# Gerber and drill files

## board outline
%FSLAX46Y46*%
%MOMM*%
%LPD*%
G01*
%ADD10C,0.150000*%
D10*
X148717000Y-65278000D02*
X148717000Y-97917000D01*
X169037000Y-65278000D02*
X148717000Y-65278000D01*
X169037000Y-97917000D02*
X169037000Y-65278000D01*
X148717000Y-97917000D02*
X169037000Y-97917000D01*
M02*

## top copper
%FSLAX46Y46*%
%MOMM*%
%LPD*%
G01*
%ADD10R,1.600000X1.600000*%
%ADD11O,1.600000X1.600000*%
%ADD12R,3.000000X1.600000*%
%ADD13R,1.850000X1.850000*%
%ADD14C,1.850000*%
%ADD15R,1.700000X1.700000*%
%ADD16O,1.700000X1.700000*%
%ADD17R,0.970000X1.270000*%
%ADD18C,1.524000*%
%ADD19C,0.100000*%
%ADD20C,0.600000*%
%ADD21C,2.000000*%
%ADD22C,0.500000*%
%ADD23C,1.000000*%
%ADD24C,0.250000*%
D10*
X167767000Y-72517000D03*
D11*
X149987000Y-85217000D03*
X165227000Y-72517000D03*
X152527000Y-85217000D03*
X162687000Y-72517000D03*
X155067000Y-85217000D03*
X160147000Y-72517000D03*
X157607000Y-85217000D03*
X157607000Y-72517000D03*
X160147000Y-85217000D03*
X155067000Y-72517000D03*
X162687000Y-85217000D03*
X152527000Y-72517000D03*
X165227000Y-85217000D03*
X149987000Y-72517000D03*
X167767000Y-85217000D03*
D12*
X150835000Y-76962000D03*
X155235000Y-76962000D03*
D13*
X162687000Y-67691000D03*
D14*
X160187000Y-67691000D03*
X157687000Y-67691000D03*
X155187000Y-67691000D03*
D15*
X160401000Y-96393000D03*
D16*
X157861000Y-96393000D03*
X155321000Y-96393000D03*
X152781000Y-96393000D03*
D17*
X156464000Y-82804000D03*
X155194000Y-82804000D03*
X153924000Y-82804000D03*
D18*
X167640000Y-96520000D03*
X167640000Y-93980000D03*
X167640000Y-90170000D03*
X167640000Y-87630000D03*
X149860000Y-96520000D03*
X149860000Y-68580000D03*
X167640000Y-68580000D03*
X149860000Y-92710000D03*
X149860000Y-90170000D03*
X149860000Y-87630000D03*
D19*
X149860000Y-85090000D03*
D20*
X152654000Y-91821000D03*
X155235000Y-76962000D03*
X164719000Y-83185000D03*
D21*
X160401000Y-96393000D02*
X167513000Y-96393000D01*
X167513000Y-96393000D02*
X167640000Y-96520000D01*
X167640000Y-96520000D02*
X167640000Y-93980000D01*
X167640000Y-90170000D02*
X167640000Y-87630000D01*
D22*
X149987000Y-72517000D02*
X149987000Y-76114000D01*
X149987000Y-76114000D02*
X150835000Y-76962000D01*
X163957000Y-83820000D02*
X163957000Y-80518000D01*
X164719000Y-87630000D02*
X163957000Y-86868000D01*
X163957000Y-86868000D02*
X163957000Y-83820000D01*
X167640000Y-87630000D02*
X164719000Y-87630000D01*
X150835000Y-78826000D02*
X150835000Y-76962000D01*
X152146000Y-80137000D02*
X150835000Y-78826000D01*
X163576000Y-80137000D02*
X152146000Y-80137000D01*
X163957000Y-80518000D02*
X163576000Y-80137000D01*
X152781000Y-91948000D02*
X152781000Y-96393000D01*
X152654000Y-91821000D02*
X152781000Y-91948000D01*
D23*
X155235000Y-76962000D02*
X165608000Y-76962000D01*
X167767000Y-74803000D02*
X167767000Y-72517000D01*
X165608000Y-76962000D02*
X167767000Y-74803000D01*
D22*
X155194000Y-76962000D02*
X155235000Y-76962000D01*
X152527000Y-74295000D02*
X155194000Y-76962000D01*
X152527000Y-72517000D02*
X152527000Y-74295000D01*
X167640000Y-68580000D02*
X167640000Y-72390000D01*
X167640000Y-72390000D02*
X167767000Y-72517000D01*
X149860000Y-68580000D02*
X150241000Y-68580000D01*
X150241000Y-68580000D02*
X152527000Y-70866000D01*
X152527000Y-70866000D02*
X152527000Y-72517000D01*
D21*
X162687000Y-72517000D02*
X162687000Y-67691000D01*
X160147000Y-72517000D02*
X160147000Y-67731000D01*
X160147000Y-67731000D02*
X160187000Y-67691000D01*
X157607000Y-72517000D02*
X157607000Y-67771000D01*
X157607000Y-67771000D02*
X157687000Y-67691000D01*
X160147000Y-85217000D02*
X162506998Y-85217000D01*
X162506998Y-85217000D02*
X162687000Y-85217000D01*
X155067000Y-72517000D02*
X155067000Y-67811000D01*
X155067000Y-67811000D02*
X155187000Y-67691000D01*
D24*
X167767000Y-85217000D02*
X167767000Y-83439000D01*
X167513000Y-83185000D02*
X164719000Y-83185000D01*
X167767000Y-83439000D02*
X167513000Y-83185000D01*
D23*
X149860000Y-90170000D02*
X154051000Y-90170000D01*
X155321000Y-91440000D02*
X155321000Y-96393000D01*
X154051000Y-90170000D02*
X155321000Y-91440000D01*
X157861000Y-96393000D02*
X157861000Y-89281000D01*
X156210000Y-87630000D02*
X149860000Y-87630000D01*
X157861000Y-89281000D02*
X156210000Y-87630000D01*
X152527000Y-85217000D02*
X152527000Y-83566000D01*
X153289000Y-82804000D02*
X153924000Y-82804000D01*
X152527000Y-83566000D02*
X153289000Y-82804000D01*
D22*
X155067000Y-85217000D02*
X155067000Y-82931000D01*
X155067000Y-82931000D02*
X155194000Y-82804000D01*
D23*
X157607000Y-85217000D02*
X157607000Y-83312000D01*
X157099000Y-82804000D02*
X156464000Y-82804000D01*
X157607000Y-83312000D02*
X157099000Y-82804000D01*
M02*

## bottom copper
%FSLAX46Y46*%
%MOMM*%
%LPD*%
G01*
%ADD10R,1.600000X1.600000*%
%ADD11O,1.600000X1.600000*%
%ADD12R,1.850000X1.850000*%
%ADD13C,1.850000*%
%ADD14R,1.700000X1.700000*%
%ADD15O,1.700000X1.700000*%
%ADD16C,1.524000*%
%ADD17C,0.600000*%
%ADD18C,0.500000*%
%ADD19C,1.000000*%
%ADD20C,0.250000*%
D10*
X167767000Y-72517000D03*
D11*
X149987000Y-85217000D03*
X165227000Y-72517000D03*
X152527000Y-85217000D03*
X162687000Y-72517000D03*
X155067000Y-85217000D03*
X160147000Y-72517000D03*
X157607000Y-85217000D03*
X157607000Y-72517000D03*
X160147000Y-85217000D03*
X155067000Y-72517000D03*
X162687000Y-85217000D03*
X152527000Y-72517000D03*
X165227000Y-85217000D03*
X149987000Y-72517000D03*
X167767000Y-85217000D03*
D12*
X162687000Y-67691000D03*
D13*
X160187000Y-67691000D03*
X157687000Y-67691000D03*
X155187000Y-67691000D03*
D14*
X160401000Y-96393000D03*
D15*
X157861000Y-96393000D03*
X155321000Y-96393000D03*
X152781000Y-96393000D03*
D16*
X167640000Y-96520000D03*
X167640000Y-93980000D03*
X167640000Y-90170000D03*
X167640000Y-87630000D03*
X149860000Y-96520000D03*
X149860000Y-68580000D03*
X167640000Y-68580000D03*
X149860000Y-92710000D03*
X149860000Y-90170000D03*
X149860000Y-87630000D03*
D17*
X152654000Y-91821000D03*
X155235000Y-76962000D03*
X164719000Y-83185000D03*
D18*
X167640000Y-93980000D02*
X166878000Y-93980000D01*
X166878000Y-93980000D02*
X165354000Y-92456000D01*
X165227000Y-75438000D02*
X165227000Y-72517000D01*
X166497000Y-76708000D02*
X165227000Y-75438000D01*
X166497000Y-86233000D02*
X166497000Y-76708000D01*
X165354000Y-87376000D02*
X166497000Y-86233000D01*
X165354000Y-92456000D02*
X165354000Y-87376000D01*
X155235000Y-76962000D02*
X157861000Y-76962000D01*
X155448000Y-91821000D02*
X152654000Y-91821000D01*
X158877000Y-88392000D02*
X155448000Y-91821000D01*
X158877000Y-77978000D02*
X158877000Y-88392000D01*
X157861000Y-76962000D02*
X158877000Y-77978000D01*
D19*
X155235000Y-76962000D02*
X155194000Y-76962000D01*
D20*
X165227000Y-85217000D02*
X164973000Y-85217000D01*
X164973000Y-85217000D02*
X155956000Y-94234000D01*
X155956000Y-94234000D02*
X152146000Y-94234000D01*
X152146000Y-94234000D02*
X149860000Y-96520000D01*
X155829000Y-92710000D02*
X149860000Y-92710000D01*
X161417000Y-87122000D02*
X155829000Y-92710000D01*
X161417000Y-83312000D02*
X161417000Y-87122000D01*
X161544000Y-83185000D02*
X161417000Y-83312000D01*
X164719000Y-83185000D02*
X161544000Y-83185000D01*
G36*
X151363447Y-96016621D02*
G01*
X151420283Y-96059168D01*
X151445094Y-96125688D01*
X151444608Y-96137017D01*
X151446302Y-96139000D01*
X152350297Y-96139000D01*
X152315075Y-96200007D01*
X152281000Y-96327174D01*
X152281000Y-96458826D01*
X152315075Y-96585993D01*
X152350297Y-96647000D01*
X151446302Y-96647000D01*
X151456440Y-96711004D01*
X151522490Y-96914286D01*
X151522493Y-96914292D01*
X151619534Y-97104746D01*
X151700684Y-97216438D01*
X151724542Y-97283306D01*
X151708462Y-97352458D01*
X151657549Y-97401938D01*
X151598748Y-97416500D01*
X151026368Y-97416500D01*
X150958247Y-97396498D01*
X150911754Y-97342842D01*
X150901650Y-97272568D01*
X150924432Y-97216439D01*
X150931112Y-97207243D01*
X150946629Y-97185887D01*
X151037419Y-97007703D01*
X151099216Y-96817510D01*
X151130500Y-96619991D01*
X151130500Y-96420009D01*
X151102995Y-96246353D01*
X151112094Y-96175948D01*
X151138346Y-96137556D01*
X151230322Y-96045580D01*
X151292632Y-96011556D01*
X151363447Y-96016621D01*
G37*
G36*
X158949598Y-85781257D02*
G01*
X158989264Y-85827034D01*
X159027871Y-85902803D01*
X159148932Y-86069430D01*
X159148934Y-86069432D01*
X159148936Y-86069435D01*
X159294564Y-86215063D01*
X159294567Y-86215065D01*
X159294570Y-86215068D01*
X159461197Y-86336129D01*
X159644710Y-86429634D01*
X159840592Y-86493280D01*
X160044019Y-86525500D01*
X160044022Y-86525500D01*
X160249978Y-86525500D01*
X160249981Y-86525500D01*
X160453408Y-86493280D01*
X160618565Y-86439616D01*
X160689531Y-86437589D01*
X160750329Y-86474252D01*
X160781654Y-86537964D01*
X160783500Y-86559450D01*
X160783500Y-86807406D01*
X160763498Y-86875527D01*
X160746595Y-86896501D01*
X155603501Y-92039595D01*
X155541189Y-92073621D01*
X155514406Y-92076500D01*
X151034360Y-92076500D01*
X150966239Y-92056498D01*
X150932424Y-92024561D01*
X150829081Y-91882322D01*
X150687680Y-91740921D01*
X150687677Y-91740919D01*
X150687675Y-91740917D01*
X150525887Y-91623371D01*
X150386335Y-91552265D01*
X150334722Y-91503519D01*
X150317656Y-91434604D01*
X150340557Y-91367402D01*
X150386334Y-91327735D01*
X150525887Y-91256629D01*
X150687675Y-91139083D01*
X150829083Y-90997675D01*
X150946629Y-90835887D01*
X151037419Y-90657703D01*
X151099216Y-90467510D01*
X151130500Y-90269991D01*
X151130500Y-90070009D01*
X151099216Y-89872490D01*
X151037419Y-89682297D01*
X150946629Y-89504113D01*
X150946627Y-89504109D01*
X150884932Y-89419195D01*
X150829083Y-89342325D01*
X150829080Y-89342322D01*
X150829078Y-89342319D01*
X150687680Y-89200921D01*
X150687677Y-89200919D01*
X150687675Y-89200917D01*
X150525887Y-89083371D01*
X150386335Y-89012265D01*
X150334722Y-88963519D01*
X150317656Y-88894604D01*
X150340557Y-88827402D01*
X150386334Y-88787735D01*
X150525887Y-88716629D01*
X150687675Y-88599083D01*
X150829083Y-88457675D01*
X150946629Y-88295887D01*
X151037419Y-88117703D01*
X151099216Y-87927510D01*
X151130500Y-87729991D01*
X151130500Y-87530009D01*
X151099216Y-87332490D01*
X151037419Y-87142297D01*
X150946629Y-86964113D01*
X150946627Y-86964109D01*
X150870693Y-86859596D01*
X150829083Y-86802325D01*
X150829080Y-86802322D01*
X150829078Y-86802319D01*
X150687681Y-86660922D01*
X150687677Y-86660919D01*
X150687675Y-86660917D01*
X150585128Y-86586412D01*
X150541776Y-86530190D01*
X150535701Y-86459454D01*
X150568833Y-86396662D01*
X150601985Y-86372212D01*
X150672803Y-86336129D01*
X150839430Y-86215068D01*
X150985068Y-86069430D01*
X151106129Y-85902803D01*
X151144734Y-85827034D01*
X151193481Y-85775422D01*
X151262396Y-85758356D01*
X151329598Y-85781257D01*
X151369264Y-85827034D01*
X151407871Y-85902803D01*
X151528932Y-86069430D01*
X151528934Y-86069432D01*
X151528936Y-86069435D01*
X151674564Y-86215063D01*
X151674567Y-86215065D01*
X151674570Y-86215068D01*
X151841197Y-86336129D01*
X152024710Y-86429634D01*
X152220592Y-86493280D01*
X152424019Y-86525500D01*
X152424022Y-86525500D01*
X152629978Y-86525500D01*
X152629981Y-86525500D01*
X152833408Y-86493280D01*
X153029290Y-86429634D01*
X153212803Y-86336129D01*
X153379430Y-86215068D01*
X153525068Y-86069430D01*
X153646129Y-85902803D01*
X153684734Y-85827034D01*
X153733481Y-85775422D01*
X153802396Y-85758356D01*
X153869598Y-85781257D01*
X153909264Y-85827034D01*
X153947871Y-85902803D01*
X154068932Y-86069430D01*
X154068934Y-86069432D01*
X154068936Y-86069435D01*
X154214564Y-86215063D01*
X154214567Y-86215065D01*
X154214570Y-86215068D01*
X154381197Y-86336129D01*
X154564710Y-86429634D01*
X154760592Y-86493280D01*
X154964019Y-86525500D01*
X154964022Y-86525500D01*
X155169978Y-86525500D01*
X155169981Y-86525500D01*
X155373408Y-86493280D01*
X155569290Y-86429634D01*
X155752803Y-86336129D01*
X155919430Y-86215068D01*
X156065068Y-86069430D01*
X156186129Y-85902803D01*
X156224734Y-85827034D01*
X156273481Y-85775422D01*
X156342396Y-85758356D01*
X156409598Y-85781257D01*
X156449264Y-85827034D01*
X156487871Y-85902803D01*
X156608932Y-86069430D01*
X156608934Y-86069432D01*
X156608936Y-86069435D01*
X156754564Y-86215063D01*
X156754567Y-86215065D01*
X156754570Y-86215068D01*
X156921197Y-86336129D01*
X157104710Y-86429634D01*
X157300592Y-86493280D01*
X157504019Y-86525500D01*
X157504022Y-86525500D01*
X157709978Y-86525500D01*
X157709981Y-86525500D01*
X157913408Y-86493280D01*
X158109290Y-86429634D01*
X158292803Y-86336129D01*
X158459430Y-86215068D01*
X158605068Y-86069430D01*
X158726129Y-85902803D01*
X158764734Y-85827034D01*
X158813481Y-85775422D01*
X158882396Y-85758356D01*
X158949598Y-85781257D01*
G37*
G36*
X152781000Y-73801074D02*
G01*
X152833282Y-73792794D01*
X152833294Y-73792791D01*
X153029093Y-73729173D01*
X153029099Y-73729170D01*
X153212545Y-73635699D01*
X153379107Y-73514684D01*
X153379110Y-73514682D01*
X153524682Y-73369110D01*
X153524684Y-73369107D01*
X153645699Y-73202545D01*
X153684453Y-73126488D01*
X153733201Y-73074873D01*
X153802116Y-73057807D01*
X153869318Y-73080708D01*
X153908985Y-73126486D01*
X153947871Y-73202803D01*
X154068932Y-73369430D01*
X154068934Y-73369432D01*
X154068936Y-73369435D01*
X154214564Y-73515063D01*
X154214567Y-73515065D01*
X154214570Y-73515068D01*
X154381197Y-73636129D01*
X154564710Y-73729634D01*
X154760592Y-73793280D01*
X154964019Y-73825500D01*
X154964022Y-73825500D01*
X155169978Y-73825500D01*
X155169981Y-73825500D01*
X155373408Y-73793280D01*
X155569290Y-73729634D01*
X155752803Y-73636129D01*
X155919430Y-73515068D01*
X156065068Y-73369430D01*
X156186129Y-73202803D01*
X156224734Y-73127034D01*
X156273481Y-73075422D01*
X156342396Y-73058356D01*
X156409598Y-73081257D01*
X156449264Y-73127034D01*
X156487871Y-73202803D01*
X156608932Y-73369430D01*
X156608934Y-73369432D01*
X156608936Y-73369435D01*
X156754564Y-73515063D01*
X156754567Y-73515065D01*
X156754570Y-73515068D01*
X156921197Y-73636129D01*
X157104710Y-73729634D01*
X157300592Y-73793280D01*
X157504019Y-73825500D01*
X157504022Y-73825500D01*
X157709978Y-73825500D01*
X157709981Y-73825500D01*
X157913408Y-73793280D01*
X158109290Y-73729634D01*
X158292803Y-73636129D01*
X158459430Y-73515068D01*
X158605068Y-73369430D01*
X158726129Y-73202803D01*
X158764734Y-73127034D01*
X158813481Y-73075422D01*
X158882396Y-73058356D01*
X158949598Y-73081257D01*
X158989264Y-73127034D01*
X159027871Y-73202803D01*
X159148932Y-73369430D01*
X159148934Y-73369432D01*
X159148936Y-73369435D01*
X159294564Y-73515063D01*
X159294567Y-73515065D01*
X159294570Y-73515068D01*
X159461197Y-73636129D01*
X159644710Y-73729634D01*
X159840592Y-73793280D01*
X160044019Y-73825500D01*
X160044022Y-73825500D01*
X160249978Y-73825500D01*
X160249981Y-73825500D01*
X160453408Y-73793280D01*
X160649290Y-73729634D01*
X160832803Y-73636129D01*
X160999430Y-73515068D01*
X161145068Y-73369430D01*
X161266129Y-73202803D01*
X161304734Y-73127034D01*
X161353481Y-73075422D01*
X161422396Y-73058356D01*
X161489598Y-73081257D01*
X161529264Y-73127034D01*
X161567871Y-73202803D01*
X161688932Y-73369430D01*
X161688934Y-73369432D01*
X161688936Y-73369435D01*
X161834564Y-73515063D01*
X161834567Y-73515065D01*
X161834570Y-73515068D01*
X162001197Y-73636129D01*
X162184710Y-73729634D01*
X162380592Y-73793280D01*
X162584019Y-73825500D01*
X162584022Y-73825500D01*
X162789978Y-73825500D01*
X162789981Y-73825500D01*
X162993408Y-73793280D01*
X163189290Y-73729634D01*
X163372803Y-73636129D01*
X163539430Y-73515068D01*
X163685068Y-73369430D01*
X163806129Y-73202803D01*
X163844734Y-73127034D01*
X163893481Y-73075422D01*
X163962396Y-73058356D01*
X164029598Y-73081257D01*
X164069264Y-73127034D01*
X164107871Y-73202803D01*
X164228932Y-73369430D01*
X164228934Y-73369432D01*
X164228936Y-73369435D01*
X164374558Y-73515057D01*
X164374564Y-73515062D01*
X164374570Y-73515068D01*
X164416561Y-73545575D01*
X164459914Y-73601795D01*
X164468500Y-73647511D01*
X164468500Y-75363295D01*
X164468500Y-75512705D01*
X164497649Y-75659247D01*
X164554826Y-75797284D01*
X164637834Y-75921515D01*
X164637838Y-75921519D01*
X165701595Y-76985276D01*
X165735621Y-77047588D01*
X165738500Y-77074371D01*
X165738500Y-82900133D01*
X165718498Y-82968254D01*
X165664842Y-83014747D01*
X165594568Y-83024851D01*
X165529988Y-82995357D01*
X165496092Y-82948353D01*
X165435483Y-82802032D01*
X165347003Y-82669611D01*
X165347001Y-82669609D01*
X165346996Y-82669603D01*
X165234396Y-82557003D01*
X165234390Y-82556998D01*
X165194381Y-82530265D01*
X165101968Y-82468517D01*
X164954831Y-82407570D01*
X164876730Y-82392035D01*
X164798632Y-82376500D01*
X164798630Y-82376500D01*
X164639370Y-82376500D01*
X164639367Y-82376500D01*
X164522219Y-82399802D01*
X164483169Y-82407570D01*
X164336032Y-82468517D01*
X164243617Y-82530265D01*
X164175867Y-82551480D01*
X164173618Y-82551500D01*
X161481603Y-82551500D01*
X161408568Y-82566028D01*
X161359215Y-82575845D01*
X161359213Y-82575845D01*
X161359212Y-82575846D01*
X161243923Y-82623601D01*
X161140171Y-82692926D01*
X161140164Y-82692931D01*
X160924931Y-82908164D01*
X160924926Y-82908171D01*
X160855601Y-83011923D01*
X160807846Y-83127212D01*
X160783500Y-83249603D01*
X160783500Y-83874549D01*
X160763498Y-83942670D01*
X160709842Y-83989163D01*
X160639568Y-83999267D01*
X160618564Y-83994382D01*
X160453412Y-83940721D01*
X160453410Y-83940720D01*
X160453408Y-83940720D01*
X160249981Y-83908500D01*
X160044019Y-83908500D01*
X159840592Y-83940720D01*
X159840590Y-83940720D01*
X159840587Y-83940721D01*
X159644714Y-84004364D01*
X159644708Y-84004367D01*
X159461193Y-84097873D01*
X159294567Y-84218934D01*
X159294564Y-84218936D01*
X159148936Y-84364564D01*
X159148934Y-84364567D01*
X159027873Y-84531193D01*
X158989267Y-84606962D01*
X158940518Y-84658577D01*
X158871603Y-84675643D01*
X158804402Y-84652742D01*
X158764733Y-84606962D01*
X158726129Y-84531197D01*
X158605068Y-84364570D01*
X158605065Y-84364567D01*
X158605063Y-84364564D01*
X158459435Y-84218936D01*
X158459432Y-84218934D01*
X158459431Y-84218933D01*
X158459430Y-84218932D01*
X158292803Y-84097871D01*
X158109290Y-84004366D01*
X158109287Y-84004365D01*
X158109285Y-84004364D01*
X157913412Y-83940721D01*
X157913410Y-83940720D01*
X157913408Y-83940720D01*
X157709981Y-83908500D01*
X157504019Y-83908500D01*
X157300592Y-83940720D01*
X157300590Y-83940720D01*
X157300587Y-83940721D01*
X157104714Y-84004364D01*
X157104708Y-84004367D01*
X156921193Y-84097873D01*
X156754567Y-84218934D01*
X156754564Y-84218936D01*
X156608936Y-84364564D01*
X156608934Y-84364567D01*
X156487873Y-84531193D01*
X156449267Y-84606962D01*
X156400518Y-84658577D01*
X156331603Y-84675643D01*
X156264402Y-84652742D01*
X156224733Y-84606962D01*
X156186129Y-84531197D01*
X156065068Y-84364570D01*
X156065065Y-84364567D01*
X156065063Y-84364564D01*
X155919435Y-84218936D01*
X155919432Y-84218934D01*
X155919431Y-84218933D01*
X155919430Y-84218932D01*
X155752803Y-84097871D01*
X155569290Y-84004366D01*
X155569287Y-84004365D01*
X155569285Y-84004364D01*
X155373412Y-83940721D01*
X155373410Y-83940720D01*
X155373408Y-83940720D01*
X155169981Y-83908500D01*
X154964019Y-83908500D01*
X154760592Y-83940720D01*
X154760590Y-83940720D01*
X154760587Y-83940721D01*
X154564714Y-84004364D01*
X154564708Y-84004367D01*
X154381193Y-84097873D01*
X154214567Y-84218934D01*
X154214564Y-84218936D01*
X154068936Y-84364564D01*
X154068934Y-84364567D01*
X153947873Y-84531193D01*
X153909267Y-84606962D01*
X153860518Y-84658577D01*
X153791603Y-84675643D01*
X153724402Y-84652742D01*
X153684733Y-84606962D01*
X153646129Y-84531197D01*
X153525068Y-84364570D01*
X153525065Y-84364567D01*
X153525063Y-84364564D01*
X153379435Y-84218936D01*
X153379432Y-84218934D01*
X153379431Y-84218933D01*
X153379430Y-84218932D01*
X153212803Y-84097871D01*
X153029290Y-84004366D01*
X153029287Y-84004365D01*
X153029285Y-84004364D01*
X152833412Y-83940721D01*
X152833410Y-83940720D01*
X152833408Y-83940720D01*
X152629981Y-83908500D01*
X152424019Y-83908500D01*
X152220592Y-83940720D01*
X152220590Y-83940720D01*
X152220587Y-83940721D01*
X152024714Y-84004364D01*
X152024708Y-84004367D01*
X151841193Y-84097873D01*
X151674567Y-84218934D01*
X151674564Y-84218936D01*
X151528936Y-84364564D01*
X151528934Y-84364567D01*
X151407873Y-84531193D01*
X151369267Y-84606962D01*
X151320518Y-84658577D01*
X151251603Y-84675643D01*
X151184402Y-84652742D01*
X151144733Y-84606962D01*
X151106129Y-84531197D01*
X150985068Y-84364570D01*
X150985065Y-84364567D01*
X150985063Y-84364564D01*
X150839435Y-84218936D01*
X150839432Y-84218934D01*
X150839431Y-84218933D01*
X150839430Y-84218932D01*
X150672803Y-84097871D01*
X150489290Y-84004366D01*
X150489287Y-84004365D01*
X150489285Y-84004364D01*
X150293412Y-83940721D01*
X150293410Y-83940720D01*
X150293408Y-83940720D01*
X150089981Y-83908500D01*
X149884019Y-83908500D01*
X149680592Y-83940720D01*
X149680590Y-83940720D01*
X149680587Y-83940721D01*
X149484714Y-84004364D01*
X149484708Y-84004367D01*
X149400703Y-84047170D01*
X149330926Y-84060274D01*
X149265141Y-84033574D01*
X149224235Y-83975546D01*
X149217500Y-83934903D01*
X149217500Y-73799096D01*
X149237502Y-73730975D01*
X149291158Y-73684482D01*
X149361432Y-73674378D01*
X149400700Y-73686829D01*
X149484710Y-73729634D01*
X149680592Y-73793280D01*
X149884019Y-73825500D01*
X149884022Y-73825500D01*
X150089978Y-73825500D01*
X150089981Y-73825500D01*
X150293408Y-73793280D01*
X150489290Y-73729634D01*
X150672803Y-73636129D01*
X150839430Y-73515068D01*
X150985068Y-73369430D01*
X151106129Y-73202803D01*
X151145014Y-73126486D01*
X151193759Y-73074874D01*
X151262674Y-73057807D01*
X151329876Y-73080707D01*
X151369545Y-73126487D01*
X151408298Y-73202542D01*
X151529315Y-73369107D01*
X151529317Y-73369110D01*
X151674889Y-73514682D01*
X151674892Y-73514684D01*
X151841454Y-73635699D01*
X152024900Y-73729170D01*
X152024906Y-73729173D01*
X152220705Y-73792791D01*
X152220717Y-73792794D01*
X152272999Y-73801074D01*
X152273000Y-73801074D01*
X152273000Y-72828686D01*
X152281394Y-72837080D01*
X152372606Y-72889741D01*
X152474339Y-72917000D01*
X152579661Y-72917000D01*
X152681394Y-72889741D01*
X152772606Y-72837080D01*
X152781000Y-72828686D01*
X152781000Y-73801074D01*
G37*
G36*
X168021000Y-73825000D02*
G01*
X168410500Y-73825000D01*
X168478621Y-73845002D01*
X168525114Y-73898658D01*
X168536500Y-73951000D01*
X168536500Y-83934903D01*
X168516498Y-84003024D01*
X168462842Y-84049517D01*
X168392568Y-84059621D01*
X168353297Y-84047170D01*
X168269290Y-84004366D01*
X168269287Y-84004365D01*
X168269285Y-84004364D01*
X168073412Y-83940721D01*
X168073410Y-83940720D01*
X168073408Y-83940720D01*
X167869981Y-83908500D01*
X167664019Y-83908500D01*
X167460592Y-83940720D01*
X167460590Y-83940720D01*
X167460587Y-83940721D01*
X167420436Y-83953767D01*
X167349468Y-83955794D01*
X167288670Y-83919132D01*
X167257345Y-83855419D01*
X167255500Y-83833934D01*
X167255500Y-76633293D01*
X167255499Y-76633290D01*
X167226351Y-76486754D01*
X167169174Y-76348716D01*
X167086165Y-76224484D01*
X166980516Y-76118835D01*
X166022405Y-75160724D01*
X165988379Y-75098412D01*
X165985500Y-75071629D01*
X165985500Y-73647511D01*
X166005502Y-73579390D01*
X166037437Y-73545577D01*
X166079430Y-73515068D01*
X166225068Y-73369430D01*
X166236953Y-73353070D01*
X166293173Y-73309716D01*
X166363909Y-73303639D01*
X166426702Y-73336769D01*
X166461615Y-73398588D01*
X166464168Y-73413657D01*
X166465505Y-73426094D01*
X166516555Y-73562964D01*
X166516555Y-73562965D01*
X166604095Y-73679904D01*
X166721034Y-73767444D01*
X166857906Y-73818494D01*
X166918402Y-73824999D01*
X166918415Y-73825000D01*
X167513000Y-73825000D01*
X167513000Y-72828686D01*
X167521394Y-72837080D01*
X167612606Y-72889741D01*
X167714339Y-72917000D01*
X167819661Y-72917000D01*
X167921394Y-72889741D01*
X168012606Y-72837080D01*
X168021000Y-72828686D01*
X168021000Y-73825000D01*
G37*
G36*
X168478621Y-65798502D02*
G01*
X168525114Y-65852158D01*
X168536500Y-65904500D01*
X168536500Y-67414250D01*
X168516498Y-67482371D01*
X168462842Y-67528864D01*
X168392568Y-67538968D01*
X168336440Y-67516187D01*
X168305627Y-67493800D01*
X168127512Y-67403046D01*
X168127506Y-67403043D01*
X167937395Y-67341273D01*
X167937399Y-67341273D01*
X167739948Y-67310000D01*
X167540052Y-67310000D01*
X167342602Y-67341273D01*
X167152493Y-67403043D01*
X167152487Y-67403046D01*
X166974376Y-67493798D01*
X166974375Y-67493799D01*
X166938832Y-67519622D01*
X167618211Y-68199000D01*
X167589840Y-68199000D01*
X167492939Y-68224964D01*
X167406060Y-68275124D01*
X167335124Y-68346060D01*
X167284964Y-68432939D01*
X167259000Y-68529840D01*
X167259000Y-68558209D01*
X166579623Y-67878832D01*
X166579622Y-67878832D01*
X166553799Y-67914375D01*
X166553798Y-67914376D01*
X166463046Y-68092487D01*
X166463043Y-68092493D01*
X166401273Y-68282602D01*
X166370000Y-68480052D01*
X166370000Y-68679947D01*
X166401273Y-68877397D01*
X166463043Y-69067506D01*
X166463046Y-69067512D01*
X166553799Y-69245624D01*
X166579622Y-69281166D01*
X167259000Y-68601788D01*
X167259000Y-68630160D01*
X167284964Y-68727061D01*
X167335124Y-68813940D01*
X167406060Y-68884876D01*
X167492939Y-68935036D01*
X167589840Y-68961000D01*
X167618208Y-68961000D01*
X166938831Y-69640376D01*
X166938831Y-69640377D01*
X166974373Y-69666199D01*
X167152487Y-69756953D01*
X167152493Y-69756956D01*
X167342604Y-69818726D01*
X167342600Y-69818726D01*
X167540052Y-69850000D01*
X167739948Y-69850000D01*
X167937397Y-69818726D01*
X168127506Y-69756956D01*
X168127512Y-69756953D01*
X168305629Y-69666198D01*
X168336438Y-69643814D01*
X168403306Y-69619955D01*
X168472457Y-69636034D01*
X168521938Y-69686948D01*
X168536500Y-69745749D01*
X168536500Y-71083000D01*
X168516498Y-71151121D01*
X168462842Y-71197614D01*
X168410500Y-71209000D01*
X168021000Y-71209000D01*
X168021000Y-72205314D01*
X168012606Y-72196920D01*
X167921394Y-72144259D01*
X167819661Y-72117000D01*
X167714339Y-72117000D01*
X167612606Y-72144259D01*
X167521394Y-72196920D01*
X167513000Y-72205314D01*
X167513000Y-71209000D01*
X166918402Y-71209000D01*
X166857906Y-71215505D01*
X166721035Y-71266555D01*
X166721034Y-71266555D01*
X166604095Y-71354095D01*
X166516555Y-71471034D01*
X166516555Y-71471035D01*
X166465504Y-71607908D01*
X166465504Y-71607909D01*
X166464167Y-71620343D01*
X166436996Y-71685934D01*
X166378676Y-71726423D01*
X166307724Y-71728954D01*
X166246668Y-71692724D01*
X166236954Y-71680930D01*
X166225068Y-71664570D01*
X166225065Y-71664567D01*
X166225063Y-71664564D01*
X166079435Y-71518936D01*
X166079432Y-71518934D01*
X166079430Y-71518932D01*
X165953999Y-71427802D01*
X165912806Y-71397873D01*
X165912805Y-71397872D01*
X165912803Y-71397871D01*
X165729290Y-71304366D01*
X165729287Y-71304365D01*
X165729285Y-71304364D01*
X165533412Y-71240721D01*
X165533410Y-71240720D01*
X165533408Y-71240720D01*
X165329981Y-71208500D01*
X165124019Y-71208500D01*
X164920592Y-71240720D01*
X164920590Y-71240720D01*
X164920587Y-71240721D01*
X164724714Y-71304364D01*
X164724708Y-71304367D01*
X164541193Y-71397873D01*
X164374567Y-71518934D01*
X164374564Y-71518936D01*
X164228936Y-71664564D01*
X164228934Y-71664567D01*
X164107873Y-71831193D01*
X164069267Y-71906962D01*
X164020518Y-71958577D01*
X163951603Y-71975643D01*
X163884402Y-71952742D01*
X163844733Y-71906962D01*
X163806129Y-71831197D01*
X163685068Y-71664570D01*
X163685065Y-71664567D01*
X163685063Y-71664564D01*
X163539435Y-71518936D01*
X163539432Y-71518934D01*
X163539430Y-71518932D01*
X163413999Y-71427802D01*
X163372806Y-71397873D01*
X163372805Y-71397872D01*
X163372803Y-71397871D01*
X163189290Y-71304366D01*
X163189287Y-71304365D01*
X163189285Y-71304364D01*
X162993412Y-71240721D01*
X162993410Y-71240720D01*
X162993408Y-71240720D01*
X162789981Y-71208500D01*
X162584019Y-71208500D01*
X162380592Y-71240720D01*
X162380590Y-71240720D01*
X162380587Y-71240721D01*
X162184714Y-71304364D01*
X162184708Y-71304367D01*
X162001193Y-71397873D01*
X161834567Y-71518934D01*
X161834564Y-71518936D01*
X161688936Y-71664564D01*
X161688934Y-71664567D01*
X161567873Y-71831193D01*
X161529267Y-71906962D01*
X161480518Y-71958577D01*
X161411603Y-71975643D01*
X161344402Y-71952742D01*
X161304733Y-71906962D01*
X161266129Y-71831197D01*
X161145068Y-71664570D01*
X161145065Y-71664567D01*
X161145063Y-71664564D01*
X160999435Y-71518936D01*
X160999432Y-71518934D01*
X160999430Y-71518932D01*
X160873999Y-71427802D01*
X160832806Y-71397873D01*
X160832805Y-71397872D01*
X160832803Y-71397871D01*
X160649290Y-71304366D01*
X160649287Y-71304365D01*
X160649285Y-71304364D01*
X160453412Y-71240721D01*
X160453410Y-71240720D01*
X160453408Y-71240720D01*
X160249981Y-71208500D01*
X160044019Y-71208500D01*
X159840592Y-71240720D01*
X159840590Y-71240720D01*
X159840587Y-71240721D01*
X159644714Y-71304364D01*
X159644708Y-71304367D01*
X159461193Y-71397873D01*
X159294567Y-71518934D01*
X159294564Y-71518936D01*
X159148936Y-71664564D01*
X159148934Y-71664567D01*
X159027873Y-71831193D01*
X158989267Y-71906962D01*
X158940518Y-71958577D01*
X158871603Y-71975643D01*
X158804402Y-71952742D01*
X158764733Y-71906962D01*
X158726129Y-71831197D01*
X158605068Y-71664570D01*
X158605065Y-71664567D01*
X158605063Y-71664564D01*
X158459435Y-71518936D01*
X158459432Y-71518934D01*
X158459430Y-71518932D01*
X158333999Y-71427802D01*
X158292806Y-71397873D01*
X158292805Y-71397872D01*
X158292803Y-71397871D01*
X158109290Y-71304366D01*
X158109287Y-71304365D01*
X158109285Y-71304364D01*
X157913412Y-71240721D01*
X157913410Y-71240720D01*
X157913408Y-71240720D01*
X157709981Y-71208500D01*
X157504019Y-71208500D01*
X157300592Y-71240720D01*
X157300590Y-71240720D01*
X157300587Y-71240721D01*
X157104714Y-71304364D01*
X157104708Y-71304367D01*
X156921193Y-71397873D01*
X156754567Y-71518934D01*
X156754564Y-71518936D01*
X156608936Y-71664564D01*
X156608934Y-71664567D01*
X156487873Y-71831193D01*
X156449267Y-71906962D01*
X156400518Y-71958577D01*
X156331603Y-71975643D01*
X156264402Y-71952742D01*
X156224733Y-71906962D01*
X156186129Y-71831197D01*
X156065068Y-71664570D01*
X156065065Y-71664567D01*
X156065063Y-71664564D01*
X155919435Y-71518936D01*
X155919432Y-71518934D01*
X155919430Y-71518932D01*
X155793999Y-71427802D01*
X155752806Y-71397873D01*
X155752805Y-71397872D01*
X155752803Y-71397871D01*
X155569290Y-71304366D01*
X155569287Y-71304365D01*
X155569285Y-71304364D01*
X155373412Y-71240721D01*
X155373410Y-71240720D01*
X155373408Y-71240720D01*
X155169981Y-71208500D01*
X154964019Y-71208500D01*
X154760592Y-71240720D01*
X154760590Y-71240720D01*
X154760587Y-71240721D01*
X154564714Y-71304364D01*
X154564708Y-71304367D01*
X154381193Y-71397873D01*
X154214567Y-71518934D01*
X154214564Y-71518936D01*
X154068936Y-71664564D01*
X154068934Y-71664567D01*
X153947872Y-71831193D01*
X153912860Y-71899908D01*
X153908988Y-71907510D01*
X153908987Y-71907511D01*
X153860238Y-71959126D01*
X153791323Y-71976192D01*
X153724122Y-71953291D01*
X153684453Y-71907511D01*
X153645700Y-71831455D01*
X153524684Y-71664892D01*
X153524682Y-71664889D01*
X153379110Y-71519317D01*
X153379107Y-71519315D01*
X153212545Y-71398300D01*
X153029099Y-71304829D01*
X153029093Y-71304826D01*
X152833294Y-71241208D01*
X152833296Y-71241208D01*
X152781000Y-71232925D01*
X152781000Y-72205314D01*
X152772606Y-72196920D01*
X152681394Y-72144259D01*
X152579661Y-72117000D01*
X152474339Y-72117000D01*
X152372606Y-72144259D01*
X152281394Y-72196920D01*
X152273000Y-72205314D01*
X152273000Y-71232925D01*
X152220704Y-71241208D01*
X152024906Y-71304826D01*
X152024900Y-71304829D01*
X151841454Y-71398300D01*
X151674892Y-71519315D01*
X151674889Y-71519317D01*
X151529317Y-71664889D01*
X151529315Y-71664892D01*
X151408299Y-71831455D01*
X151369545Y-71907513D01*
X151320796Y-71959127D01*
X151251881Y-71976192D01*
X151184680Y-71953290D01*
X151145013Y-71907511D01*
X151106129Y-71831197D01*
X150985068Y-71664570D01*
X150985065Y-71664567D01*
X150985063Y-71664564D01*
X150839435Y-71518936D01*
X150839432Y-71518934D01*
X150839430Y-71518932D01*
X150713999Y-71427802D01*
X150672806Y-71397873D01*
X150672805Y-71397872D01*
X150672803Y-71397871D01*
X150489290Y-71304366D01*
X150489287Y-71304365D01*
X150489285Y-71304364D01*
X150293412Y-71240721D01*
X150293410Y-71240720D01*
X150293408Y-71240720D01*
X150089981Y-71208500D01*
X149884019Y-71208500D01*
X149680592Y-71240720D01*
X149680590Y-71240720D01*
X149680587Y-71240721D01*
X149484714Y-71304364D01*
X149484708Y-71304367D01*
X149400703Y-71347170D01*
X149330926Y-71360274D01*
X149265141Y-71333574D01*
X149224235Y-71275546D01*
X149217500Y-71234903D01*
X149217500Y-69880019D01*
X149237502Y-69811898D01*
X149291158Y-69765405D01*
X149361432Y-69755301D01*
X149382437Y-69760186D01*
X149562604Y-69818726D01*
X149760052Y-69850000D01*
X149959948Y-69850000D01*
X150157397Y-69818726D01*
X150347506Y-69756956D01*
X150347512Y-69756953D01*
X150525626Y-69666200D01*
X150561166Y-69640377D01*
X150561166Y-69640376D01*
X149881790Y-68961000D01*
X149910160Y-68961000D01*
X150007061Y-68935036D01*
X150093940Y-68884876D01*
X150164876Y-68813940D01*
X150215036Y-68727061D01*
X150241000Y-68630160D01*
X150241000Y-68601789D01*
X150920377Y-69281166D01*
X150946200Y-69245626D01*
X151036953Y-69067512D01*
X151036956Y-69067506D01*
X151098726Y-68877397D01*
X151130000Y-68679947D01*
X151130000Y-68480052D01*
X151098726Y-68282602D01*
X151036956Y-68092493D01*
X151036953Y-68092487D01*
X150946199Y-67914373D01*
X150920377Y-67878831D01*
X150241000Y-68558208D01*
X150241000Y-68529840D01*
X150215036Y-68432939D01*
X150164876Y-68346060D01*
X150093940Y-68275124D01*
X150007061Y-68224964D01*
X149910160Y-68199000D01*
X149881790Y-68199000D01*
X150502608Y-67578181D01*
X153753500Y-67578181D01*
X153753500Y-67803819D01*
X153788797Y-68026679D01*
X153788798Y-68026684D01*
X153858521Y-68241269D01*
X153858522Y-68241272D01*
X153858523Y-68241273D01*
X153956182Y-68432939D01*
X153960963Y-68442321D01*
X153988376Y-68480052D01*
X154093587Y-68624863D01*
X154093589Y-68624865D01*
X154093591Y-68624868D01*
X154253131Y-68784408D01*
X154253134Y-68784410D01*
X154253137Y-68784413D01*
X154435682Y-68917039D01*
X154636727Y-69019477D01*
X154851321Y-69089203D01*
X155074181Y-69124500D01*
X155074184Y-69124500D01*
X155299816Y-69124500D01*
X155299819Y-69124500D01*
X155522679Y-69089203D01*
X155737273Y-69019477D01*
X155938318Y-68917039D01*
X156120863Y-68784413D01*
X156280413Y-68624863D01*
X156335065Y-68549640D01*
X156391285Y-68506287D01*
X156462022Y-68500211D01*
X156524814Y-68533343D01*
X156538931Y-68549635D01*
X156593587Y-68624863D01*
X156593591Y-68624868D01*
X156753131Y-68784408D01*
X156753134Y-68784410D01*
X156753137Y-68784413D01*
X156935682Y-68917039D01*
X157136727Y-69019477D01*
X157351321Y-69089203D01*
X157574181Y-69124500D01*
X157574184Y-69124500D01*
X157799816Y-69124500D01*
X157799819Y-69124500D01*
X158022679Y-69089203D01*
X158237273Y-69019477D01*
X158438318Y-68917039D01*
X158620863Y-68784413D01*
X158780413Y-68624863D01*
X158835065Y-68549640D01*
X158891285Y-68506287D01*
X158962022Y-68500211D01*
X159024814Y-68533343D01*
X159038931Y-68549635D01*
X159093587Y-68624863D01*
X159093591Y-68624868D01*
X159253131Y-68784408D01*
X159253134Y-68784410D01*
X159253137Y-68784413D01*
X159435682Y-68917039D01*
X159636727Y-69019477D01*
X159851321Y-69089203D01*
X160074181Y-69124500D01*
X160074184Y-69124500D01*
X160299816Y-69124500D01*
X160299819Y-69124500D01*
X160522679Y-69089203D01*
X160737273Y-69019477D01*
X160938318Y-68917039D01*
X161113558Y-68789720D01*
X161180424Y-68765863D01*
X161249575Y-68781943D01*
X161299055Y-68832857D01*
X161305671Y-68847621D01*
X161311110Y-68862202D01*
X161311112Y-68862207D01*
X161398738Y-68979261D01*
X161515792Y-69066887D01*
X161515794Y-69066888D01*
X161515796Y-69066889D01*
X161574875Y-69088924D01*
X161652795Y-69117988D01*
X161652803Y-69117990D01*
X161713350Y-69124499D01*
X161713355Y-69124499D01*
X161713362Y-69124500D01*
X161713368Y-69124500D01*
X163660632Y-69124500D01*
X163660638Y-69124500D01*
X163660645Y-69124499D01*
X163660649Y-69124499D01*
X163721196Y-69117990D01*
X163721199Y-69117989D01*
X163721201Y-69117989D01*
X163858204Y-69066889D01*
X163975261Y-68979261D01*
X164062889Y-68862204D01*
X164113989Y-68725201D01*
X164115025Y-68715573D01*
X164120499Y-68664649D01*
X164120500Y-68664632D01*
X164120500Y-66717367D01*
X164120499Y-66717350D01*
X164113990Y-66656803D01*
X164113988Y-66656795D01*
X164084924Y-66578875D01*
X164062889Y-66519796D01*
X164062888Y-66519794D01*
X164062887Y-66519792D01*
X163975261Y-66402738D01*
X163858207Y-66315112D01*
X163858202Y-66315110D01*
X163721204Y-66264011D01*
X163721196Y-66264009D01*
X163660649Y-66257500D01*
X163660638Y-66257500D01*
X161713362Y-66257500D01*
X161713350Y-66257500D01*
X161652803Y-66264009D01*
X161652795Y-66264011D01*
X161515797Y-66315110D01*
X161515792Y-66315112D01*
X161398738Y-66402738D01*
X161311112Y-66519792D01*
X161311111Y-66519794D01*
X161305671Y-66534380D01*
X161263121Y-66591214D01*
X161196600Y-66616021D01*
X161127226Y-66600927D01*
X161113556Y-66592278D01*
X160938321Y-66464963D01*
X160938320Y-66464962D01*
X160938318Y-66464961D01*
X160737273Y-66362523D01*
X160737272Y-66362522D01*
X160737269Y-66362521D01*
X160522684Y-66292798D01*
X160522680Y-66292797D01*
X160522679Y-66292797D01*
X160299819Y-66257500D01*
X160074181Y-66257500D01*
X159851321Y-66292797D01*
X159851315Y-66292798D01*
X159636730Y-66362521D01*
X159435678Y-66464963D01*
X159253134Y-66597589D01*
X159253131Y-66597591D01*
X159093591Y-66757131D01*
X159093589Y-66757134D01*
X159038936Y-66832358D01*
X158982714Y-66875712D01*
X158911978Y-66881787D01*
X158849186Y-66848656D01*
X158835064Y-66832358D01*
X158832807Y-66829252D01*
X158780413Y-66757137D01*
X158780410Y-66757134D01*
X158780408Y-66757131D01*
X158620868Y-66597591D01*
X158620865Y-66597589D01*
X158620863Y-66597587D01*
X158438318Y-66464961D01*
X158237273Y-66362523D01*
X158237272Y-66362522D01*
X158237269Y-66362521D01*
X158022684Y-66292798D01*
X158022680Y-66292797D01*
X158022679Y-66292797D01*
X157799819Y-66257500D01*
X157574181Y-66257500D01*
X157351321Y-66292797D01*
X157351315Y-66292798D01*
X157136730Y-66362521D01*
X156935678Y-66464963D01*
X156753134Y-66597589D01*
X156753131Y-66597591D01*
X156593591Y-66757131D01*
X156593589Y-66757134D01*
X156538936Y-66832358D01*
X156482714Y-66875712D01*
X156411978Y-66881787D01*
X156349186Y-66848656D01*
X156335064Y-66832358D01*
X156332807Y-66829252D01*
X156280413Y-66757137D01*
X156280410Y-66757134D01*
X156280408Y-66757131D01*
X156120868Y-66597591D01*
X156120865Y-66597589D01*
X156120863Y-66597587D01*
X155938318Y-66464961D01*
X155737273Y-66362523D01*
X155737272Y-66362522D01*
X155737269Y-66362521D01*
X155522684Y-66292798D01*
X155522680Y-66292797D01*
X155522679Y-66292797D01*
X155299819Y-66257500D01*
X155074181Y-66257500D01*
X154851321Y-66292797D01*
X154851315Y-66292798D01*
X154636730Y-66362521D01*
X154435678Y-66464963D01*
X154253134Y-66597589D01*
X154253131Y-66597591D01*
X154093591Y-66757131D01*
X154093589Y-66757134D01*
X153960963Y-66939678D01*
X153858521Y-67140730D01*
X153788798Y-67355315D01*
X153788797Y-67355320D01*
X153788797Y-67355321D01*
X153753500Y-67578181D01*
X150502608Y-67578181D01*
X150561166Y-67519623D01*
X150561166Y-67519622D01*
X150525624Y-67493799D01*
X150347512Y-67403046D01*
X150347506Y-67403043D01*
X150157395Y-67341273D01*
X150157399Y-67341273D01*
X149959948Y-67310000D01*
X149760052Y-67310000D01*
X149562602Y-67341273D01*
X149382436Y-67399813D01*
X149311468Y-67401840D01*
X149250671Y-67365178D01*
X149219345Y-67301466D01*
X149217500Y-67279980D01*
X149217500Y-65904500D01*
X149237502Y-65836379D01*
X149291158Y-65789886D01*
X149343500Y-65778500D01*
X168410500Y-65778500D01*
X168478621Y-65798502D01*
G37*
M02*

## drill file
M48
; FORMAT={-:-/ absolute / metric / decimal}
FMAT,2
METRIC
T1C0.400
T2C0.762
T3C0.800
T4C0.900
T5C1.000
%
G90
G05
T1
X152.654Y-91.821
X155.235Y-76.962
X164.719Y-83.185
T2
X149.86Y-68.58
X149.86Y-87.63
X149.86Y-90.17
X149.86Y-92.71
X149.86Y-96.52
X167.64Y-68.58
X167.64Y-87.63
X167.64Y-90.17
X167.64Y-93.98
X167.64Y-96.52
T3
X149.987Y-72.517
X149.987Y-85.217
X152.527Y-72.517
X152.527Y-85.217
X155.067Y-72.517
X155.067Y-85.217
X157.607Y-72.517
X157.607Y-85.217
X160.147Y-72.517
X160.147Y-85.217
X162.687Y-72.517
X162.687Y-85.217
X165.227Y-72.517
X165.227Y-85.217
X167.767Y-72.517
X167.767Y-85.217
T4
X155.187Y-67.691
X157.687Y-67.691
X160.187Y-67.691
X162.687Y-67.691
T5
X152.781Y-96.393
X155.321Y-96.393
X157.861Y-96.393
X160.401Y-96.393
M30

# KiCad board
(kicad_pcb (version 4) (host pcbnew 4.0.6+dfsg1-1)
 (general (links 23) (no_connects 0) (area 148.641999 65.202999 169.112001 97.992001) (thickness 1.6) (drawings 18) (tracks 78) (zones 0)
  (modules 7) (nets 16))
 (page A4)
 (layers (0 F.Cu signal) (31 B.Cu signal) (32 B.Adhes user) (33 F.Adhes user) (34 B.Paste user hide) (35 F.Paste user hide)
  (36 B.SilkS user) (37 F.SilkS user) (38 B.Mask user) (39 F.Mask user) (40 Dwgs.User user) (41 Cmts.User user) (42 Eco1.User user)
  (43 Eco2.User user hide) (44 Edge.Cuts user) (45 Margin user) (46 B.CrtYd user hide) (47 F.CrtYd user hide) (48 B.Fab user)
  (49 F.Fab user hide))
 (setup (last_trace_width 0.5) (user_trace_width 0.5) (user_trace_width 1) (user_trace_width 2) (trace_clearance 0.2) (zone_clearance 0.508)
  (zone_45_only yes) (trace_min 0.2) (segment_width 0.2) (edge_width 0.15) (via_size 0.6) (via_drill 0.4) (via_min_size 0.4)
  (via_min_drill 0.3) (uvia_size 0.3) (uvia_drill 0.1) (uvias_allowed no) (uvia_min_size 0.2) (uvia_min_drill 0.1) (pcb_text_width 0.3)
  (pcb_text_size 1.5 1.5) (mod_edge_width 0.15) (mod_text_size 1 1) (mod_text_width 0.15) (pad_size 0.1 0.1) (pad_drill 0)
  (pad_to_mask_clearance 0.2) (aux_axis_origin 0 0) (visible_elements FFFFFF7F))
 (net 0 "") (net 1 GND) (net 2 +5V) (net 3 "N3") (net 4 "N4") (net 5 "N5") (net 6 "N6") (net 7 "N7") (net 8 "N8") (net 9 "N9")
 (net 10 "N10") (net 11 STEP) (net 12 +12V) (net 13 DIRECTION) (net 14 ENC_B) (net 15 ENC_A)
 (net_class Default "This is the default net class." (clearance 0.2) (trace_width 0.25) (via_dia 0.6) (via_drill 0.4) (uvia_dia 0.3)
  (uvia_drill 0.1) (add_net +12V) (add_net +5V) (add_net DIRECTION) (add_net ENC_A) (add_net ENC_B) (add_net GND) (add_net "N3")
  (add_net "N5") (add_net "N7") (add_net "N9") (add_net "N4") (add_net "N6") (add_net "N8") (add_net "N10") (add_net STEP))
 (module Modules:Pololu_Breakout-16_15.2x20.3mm (layer F.Cu) (at 167.767 72.517 270)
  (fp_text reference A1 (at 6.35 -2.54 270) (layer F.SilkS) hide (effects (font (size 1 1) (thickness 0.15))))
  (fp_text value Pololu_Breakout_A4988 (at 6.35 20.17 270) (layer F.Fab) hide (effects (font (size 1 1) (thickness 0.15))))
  (pad 1 thru_hole rect (at 0 0 270) (size 1.6 1.6) (drill 0.8) (layers *.Cu *.Mask) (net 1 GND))
  (pad 9 thru_hole oval (at 12.7 17.78 270) (size 1.6 1.6) (drill 0.8) (layers *.Cu *.Mask))
  (pad 2 thru_hole oval (at 0 2.54 270) (size 1.6 1.6) (drill 0.8) (layers *.Cu *.Mask) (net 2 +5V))
  (pad 10 thru_hole oval (at 12.7 15.24 270) (size 1.6 1.6) (drill 0.8) (layers *.Cu *.Mask) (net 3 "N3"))
  (pad 3 thru_hole oval (at 0 5.08 270) (size 1.6 1.6) (drill 0.8) (layers *.Cu *.Mask) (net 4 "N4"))
  (pad 11 thru_hole oval (at 12.7 12.7 270) (size 1.6 1.6) (drill 0.8) (layers *.Cu *.Mask) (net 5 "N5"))
  (pad 4 thru_hole oval (at 0 7.62 270) (size 1.6 1.6) (drill 0.8) (layers *.Cu *.Mask) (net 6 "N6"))
  (pad 12 thru_hole oval (at 12.7 10.16 270) (size 1.6 1.6) (drill 0.8) (layers *.Cu *.Mask) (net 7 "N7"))
  (pad 5 thru_hole oval (at 0 10.16 270) (size 1.6 1.6) (drill 0.8) (layers *.Cu *.Mask) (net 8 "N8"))
  (pad 13 thru_hole oval (at 12.7 7.62 270) (size 1.6 1.6) (drill 0.8) (layers *.Cu *.Mask) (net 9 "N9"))
  (pad 6 thru_hole oval (at 0 12.7 270) (size 1.6 1.6) (drill 0.8) (layers *.Cu *.Mask) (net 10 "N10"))
  (pad 14 thru_hole oval (at 12.7 5.08 270) (size 1.6 1.6) (drill 0.8) (layers *.Cu *.Mask) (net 9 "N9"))
  (pad 7 thru_hole oval (at 0 15.24 270) (size 1.6 1.6) (drill 0.8) (layers *.Cu *.Mask) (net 1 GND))
  (pad 15 thru_hole oval (at 12.7 2.54 270) (size 1.6 1.6) (drill 0.8) (layers *.Cu *.Mask) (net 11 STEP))
  (pad 8 thru_hole oval (at 0 17.78 270) (size 1.6 1.6) (drill 0.8) (layers *.Cu *.Mask) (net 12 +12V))
  (pad 16 thru_hole oval (at 12.7 0 270) (size 1.6 1.6) (drill 0.8) (layers *.Cu *.Mask) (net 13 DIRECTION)))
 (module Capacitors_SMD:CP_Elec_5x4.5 (layer F.Cu) (at 153.035 76.962)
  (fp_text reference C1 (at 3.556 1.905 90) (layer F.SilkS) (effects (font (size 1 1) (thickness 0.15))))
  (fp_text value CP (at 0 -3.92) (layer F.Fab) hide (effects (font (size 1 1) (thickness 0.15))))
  (pad 1 smd rect (at -2.2 0 180) (size 3 1.6) (layers F.Cu F.Paste F.Mask) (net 12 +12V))
  (pad 2 smd rect (at 2.2 0 180) (size 3 1.6) (layers F.Cu F.Paste F.Mask) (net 1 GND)))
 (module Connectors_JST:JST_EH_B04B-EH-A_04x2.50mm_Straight (layer F.Cu) (at 162.687 67.691 180)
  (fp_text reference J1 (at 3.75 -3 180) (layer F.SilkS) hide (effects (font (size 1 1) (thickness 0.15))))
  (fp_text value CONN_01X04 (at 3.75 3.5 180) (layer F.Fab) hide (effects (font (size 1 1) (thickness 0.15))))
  (pad 1 thru_hole rect (at 0 0 180) (size 1.85 1.85) (drill 0.9) (layers *.Cu *.Mask) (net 4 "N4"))
  (pad 2 thru_hole circle (at 2.5 0 180) (size 1.85 1.85) (drill 0.9) (layers *.Cu *.Mask) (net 6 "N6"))
  (pad 3 thru_hole circle (at 5 0 180) (size 1.85 1.85) (drill 0.9) (layers *.Cu *.Mask) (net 8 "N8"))
  (pad 4 thru_hole circle (at 7.5 0 180) (size 1.85 1.85) (drill 0.9) (layers *.Cu *.Mask) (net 10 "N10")))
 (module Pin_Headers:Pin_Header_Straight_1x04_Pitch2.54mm (layer F.Cu) (at 160.401 96.393 270)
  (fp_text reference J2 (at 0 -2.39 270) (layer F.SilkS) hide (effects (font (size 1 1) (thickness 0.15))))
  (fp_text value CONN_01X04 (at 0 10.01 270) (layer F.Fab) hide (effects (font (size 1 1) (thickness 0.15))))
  (pad 1 thru_hole rect (at 0 0 270) (size 1.7 1.7) (drill 1) (layers *.Cu *.Mask) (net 2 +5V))
  (pad 2 thru_hole oval (at 0 2.54 270) (size 1.7 1.7) (drill 1) (layers *.Cu *.Mask) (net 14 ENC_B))
  (pad 3 thru_hole oval (at 0 5.08 270) (size 1.7 1.7) (drill 1) (layers *.Cu *.Mask) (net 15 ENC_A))
  (pad 4 thru_hole oval (at 0 7.62 270) (size 1.7 1.7) (drill 1) (layers *.Cu *.Mask) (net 1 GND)))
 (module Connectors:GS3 (layer F.Cu) (at 155.194 82.804 270)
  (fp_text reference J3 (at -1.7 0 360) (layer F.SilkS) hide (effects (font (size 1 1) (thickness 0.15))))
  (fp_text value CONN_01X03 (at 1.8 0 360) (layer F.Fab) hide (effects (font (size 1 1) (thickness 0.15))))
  (pad 1 smd rect (at 0 -1.27 270) (size 1.27 0.97) (layers F.Cu F.Paste F.Mask) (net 7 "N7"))
  (pad 2 smd rect (at 0 0 270) (size 1.27 0.97) (layers F.Cu F.Paste F.Mask) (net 5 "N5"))
  (pad 3 smd rect (at 0 1.27 270) (size 1.27 0.97) (layers F.Cu F.Paste F.Mask) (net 3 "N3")))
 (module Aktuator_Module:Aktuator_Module (layer F.Cu) (at 148.59 97.79)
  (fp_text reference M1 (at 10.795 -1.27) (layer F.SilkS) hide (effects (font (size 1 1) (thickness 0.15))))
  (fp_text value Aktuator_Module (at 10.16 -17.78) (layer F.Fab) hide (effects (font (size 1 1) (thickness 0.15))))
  (pad 1 thru_hole circle (at 19.05 -1.27) (size 1.524 1.524) (drill 0.762) (layers *.Cu *.Mask) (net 2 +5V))
  (pad 1 thru_hole circle (at 19.05 -3.81) (size 1.524 1.524) (drill 0.762) (layers *.Cu *.Mask) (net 2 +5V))
  (pad 2 thru_hole circle (at 19.05 -7.62) (size 1.524 1.524) (drill 0.762) (layers *.Cu *.Mask) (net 12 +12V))
  (pad 2 thru_hole circle (at 19.05 -10.16) (size 1.524 1.524) (drill 0.762) (layers *.Cu *.Mask) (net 12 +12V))
  (pad 3 thru_hole circle (at 1.27 -1.27) (size 1.524 1.524) (drill 0.762) (layers *.Cu *.Mask) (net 11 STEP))
  (pad 4 thru_hole circle (at 1.27 -29.21) (size 1.524 1.524) (drill 0.762) (layers *.Cu *.Mask) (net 1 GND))
  (pad 4 thru_hole circle (at 19.05 -29.21) (size 1.524 1.524) (drill 0.762) (layers *.Cu *.Mask) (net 1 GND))
  (pad 6 thru_hole circle (at 1.27 -5.08) (size 1.524 1.524) (drill 0.762) (layers *.Cu *.Mask) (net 13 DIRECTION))
  (pad 7 thru_hole circle (at 1.27 -7.62) (size 1.524 1.524) (drill 0.762) (layers *.Cu *.Mask) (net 15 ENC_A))
  (pad 8 thru_hole circle (at 1.27 -10.16) (size 1.524 1.524) (drill 0.762) (layers *.Cu *.Mask) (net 14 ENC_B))
  (pad 9 smd circle (at 1.27 -12.7) (size 0.1 0.1) (layers F.Cu F.Paste F.Mask)))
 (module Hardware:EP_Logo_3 (layer F.Cu) (at 162.56 78.359)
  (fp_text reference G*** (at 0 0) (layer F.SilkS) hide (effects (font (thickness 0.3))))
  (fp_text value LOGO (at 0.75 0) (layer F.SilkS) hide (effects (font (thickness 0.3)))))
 (gr_line (start 148.717 65.278) (end 148.717 97.917) (angle 90) (layer Edge.Cuts) (width 0.15))
 (gr_line (start 169.037 65.278) (end 148.717 65.278) (angle 90) (layer Edge.Cuts) (width 0.15))
 (gr_line (start 169.037 97.917) (end 169.037 65.278) (angle 90) (layer Edge.Cuts) (width 0.15))
 (gr_line (start 148.717 97.917) (end 169.037 97.917) (angle 90) (layer Edge.Cuts) (width 0.15))
 (segment (start 167.64 93.98) (end 166.878 93.98) (width 0.5) (layer B.Cu) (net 2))
 (segment (start 166.878 93.98) (end 165.354 92.456) (width 0.5) (layer B.Cu) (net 2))
 (segment (start 165.227 75.438) (end 165.227 72.517) (width 0.5) (layer B.Cu) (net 2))
 (segment (start 166.497 76.708) (end 165.227 75.438) (width 0.5) (layer B.Cu) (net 2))
 (segment (start 166.497 86.233) (end 166.497 76.708) (width 0.5) (layer B.Cu) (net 2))
 (segment (start 165.354 87.376) (end 166.497 86.233) (width 0.5) (layer B.Cu) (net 2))
 (segment (start 165.354 92.456) (end 165.354 87.376) (width 0.5) (layer B.Cu) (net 2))
 (segment (start 160.401 96.393) (end 167.513 96.393) (width 2) (layer F.Cu) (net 2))
 (segment (start 167.513 96.393) (end 167.64 96.52) (width 2) (layer F.Cu) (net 2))
 (segment (start 167.64 96.52) (end 167.64 93.98) (width 2) (layer F.Cu) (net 2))
 (segment (start 167.64 90.17) (end 167.64 87.63) (width 2) (layer F.Cu) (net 12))
 (segment (start 149.987 72.517) (end 149.987 76.114) (width 0.5) (layer F.Cu) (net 12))
 (segment (start 149.987 76.114) (end 150.835 76.962) (width 0.5) (layer F.Cu) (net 12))
 (segment (start 163.957 83.82) (end 163.957 80.518) (width 0.5) (layer F.Cu) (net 12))
 (segment (start 164.719 87.63) (end 163.957 86.868) (width 0.5) (layer F.Cu) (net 12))
 (segment (start 163.957 86.868) (end 163.957 83.82) (width 0.5) (layer F.Cu) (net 12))
 (segment (start 167.64 87.63) (end 164.719 87.63) (width 0.5) (layer F.Cu) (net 12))
 (segment (start 150.835 78.826) (end 150.835 76.962) (width 0.5) (layer F.Cu) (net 12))
 (segment (start 152.146 80.137) (end 150.835 78.826) (width 0.5) (layer F.Cu) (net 12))
 (segment (start 163.576 80.137) (end 152.146 80.137) (width 0.5) (layer F.Cu) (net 12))
 (segment (start 163.957 80.518) (end 163.576 80.137) (width 0.5) (layer F.Cu) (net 12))
 (segment (start 155.235 76.962) (end 157.861 76.962) (width 0.5) (layer B.Cu) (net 1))
 (segment (start 152.781 91.948) (end 152.781 96.393) (width 0.5) (layer F.Cu) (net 1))
 (segment (start 152.654 91.821) (end 152.781 91.948) (width 0.5) (layer F.Cu) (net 1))
 (via (at 152.654 91.821) (size 0.6) (drill 0.4) (layers F.Cu B.Cu) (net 1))
 (segment (start 155.448 91.821) (end 152.654 91.821) (width 0.5) (layer B.Cu) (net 1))
 (segment (start 158.877 88.392) (end 155.448 91.821) (width 0.5) (layer B.Cu) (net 1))
 (segment (start 158.877 77.978) (end 158.877 88.392) (width 0.5) (layer B.Cu) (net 1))
 (segment (start 157.861 76.962) (end 158.877 77.978) (width 0.5) (layer B.Cu) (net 1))
 (segment (start 155.235 76.962) (end 165.608 76.962) (width 1) (layer F.Cu) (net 1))
 (segment (start 167.767 74.803) (end 167.767 72.517) (width 1) (layer F.Cu) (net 1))
 (segment (start 165.608 76.962) (end 167.767 74.803) (width 1) (layer F.Cu) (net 1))
 (via (at 155.235 76.962) (size 0.6) (drill 0.4) (layers F.Cu B.Cu) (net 1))
 (segment (start 155.194 76.962) (end 155.235 76.962) (width 0.5) (layer F.Cu) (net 1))
 (segment (start 152.527 74.295) (end 155.194 76.962) (width 0.5) (layer F.Cu) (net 1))
 (segment (start 152.527 72.517) (end 152.527 74.295) (width 0.5) (layer F.Cu) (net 1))
 (segment (start 155.235 76.962) (end 155.194 76.962) (width 1) (layer B.Cu) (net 1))
 (segment (start 167.64 68.58) (end 167.64 72.39) (width 0.5) (layer F.Cu) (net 1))
 (segment (start 167.64 72.39) (end 167.767 72.517) (width 0.5) (layer F.Cu) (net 1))
 (segment (start 149.86 68.58) (end 150.241 68.58) (width 0.5) (layer F.Cu) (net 1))
 (segment (start 150.241 68.58) (end 152.527 70.866) (width 0.5) (layer F.Cu) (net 1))
 (segment (start 152.527 70.866) (end 152.527 72.517) (width 0.5) (layer F.Cu) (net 1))
 (segment (start 162.687 72.517) (end 162.687 67.691) (width 2) (layer F.Cu) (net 4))
 (segment (start 160.147 72.517) (end 160.147 67.731) (width 2) (layer F.Cu) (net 6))
 (segment (start 160.147 67.731) (end 160.187 67.691) (width 2) (layer F.Cu) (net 6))
 (segment (start 157.607 72.517) (end 157.607 67.771) (width 2) (layer F.Cu) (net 8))
 (segment (start 157.607 67.771) (end 157.687 67.691) (width 2) (layer F.Cu) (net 8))
 (segment (start 160.147 85.217) (end 162.506998 85.217) (width 2) (layer F.Cu) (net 9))
 (segment (start 162.506998 85.217) (end 162.687 85.217) (width 2) (layer F.Cu) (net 9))
 (segment (start 155.067 72.517) (end 155.067 67.811) (width 2) (layer F.Cu) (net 10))
 (segment (start 155.067 67.811) (end 155.187 67.691) (width 2) (layer F.Cu) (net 10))
 (segment (start 165.227 85.217) (end 164.973 85.217) (width 0.25) (layer B.Cu) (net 11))
 (segment (start 164.973 85.217) (end 155.956 94.234) (width 0.25) (layer B.Cu) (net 11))
 (segment (start 155.956 94.234) (end 152.146 94.234) (width 0.25) (layer B.Cu) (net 11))
 (segment (start 152.146 94.234) (end 149.86 96.52) (width 0.25) (layer B.Cu) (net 11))
 (segment (start 167.767 85.217) (end 167.767 83.439) (width 0.25) (layer F.Cu) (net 13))
 (segment (start 155.829 92.71) (end 149.86 92.71) (width 0.25) (layer B.Cu) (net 13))
 (segment (start 161.417 87.122) (end 155.829 92.71) (width 0.25) (layer B.Cu) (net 13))
 (segment (start 161.417 83.312) (end 161.417 87.122) (width 0.25) (layer B.Cu) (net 13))
 (segment (start 161.544 83.185) (end 161.417 83.312) (width 0.25) (layer B.Cu) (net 13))
 (segment (start 164.719 83.185) (end 161.544 83.185) (width 0.25) (layer B.Cu) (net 13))
 (via (at 164.719 83.185) (size 0.6) (drill 0.4) (layers F.Cu B.Cu) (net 13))
 (segment (start 167.513 83.185) (end 164.719 83.185) (width 0.25) (layer F.Cu) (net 13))
 (segment (start 167.767 83.439) (end 167.513 83.185) (width 0.25) (layer F.Cu) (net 13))
 (segment (start 149.86 90.17) (end 154.051 90.17) (width 1) (layer F.Cu) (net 15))
 (segment (start 155.321 91.44) (end 155.321 96.393) (width 1) (layer F.Cu) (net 15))
 (segment (start 154.051 90.17) (end 155.321 91.44) (width 1) (layer F.Cu) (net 15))
 (segment (start 157.861 96.393) (end 157.861 89.281) (width 1) (layer F.Cu) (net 14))
 (segment (start 156.21 87.63) (end 149.86 87.63) (width 1) (layer F.Cu) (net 14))
 (segment (start 157.861 89.281) (end 156.21 87.63) (width 1) (layer F.Cu) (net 14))
 (segment (start 152.527 85.217) (end 152.527 83.566) (width 1) (layer F.Cu) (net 3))
 (segment (start 153.289 82.804) (end 153.924 82.804) (width 1) (layer F.Cu) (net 3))
 (segment (start 152.527 83.566) (end 153.289 82.804) (width 1) (layer F.Cu) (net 3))
 (segment (start 155.067 85.217) (end 155.067 82.931) (width 0.5) (layer F.Cu) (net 5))
 (segment (start 155.067 82.931) (end 155.194 82.804) (width 0.5) (layer F.Cu) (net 5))
 (segment (start 157.607 85.217) (end 157.607 83.312) (width 1) (layer F.Cu) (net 7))
 (segment (start 157.099 82.804) (end 156.464 82.804) (width 1) (layer F.Cu) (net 7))
 (segment (start 157.607 83.312) (end 157.099 82.804) (width 1) (layer F.Cu) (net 7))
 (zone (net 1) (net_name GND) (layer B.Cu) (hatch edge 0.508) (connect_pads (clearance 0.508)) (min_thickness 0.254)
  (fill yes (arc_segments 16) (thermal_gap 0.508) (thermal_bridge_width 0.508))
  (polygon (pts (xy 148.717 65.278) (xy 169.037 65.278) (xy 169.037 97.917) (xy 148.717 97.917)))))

